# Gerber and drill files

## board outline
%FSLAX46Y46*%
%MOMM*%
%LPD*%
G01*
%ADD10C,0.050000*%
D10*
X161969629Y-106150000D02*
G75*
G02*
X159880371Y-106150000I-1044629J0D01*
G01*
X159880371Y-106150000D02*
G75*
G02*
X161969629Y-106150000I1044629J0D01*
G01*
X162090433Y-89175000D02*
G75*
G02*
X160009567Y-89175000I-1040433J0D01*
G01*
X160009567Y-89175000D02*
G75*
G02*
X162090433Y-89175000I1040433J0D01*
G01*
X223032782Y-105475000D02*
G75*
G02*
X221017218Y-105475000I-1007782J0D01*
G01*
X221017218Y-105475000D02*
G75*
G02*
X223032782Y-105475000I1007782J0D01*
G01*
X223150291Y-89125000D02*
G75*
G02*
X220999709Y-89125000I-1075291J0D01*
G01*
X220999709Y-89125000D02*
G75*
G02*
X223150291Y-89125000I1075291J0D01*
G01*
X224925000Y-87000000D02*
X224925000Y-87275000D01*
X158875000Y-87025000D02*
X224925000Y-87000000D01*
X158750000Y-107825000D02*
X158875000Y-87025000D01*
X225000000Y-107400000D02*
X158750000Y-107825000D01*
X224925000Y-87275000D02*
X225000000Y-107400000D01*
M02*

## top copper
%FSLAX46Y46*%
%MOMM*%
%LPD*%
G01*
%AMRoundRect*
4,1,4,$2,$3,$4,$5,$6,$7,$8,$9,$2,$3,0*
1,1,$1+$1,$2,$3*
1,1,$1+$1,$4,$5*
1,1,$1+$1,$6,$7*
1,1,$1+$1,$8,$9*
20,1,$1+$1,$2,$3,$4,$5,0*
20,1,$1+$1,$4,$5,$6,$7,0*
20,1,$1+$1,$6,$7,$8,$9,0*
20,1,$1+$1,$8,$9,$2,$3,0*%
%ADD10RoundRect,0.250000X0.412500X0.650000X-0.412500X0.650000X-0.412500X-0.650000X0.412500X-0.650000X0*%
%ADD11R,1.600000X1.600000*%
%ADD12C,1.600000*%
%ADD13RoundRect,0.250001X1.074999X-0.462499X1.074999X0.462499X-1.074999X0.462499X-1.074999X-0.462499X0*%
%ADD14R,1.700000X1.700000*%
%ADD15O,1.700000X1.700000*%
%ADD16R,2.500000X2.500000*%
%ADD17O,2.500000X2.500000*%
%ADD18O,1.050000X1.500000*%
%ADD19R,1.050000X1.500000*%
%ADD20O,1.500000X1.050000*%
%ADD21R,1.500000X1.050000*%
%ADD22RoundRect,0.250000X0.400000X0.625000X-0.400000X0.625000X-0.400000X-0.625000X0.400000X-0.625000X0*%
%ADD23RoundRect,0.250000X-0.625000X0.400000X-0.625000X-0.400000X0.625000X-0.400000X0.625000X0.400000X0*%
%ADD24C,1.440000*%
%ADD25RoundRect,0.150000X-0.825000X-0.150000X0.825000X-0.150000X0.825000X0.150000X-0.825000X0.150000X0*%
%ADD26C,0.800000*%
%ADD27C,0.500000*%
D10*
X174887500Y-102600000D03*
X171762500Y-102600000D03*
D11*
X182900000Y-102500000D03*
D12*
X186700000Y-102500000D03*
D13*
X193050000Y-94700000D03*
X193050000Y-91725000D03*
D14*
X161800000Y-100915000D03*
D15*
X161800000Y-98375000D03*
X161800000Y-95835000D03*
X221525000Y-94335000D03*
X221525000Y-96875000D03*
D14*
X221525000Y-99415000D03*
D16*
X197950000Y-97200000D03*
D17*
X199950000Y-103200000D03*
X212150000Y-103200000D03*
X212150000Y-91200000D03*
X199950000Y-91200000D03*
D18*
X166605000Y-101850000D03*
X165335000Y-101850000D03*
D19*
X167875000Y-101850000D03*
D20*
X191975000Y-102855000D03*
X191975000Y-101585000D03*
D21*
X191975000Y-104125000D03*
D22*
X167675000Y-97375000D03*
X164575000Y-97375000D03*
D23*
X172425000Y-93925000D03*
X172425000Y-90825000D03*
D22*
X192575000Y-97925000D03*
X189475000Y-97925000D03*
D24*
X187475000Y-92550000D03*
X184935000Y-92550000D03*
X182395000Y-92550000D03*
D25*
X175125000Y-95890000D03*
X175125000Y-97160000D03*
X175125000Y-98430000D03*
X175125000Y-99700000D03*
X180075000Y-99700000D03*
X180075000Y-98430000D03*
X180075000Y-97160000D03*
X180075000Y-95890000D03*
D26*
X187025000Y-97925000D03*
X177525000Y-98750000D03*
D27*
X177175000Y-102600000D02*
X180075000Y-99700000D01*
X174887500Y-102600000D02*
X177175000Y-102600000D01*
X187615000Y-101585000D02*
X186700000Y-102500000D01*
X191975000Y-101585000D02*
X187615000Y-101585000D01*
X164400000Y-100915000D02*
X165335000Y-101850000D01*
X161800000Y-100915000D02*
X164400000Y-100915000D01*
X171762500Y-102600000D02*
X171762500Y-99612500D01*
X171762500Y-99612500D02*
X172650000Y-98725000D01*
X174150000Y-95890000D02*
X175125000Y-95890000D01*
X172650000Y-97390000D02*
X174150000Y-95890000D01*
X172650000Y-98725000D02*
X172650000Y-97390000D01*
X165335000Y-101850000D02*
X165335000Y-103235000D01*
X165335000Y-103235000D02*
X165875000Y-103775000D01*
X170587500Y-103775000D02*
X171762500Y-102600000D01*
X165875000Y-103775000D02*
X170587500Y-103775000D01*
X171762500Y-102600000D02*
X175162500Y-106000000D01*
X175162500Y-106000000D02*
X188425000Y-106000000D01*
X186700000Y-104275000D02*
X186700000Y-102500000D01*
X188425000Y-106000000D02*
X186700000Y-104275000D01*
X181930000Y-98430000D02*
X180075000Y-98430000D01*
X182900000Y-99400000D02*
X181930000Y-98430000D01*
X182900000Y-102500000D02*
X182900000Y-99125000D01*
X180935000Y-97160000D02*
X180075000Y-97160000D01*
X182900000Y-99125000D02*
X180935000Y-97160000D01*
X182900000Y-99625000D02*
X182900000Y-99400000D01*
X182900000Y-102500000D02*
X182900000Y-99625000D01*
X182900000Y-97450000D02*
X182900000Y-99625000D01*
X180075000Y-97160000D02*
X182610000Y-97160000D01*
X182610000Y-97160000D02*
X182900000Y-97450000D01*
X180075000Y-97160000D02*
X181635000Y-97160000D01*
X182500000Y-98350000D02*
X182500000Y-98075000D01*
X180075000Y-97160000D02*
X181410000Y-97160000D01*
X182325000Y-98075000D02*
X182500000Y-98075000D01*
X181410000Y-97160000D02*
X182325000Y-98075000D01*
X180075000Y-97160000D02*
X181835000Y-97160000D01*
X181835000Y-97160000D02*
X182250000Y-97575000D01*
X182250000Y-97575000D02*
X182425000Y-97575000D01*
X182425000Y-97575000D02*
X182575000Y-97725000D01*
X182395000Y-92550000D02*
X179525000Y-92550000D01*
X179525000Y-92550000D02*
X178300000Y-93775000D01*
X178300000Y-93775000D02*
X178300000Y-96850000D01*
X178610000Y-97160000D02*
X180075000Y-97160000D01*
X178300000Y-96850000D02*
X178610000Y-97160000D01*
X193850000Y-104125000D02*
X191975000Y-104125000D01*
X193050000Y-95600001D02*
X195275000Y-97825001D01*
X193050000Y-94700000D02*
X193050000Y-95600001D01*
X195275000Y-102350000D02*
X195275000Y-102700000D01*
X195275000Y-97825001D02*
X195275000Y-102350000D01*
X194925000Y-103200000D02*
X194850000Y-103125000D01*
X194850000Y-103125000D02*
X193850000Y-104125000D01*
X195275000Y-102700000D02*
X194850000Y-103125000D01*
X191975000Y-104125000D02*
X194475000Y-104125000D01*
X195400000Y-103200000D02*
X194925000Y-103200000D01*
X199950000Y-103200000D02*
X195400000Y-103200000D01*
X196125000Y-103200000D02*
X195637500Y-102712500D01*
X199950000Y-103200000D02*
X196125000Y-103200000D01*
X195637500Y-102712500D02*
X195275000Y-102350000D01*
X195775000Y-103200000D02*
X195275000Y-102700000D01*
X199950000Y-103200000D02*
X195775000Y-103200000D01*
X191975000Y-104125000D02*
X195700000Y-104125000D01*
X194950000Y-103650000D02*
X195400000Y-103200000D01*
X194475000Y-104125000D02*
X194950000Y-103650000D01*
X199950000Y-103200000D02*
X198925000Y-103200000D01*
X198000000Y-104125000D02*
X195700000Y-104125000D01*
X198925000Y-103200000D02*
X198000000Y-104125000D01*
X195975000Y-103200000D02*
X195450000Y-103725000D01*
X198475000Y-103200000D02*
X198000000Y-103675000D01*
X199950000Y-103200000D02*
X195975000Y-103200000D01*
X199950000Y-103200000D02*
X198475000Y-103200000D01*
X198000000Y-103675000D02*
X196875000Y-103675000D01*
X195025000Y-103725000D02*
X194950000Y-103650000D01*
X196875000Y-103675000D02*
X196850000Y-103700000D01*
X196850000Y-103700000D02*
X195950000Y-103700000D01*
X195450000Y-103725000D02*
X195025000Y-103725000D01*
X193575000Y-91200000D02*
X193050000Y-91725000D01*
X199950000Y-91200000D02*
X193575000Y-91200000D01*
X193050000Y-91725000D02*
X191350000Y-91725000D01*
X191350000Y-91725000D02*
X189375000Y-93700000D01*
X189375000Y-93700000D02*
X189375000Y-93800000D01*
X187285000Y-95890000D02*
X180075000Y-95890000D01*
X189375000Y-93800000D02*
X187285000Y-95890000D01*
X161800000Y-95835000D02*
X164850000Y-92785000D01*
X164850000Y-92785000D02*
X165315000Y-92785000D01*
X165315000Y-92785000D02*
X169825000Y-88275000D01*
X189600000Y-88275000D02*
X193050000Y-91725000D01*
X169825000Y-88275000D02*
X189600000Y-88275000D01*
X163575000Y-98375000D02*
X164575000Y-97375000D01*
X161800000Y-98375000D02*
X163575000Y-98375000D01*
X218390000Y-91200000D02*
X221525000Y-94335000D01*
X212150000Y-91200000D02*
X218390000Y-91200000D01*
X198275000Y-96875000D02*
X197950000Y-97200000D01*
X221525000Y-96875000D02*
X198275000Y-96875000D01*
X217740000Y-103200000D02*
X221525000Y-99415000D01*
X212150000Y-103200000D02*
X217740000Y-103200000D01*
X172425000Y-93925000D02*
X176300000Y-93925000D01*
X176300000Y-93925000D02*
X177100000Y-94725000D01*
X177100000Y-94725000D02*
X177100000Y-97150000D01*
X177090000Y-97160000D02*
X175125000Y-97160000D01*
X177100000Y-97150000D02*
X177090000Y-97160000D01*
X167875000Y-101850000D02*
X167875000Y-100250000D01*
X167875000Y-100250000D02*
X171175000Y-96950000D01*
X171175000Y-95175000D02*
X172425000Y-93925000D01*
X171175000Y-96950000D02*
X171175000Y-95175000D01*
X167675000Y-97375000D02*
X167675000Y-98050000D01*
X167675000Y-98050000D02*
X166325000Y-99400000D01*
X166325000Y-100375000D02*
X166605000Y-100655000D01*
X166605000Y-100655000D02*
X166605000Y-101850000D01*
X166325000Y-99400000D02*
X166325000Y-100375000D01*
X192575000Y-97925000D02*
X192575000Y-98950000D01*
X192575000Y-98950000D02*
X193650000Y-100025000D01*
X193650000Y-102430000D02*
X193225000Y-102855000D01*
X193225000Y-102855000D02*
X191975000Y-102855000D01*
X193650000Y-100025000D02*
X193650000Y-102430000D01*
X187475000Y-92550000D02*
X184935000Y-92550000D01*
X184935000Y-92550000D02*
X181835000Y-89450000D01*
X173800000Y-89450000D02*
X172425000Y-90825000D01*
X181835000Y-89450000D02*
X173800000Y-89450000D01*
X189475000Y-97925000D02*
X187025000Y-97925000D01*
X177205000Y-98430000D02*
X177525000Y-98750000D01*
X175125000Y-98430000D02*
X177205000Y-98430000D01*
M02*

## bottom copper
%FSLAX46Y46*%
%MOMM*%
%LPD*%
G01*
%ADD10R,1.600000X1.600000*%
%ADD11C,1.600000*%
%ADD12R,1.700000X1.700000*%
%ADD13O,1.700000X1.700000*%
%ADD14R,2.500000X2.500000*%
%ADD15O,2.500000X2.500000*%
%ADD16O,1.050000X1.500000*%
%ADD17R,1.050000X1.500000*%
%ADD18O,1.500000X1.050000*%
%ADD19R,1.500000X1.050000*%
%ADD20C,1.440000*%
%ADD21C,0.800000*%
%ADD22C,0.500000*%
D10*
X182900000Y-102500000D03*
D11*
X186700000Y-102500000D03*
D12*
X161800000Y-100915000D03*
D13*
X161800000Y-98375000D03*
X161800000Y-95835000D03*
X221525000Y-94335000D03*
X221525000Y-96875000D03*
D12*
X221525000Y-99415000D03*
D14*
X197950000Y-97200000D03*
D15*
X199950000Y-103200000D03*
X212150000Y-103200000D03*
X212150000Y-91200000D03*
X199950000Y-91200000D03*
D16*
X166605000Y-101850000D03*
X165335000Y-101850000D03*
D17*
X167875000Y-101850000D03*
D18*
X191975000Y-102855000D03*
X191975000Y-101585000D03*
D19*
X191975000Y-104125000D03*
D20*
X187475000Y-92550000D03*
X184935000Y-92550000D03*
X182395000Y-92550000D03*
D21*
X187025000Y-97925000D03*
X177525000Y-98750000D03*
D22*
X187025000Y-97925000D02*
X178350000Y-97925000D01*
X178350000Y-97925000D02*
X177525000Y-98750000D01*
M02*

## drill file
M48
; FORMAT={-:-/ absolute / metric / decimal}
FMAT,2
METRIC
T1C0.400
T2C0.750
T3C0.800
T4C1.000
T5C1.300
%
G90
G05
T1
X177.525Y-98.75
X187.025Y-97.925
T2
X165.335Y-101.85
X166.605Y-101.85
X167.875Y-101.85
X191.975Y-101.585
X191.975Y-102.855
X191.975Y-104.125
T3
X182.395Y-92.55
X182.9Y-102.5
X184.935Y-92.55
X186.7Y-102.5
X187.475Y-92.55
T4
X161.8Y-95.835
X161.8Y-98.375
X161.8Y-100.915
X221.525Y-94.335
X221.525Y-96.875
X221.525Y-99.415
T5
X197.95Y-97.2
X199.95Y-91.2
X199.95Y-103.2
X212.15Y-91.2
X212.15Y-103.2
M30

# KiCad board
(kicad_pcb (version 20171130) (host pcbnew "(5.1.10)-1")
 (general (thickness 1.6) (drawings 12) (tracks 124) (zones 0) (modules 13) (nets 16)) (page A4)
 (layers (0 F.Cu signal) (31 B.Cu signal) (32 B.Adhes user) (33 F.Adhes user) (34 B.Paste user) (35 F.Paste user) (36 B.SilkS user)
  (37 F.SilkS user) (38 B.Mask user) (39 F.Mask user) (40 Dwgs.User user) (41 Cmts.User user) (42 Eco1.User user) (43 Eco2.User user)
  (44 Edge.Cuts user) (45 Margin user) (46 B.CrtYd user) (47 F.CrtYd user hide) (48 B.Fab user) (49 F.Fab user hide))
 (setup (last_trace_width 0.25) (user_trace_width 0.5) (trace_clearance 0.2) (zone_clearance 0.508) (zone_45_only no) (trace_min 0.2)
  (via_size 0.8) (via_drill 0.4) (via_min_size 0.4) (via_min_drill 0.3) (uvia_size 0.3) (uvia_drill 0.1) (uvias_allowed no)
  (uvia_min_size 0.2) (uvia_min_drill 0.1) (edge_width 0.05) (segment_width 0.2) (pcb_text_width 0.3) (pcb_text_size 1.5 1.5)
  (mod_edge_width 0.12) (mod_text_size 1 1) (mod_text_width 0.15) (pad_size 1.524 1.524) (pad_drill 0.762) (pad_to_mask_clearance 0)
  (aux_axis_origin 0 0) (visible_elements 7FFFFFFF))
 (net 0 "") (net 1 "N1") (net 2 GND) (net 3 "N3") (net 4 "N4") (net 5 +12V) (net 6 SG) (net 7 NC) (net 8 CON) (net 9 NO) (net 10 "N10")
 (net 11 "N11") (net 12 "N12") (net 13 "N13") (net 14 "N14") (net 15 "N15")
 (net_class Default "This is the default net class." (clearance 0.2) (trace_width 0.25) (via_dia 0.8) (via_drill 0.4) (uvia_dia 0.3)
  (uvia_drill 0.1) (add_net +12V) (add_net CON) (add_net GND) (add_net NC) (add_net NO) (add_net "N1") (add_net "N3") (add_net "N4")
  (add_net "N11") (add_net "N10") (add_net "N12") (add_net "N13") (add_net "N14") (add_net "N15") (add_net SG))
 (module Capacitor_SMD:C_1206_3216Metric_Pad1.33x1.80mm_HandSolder (layer F.Cu) (at 173.325 102.6 180)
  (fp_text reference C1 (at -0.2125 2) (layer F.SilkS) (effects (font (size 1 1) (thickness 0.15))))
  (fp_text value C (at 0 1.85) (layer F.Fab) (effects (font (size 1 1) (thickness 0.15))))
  (pad 1 smd roundrect (at -1.5625 0 180) (size 1.325 1.8) (layers F.Cu F.Paste F.Mask) (roundrect_rratio 0.188679) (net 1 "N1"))
  (pad 2 smd roundrect (at 1.5625 0 180) (size 1.325 1.8) (layers F.Cu F.Paste F.Mask) (roundrect_rratio 0.188679) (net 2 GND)))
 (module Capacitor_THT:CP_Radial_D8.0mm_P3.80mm (layer F.Cu) (at 182.9 102.5)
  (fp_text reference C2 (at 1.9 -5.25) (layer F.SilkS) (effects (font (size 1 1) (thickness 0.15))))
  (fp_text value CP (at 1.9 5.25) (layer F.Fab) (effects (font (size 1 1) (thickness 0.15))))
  (pad 1 thru_hole rect (at 0 0) (size 1.6 1.6) (drill 0.8) (layers *.Cu *.Mask) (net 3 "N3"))
  (pad 2 thru_hole circle (at 3.8 0) (size 1.6 1.6) (drill 0.8) (layers *.Cu *.Mask) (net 2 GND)))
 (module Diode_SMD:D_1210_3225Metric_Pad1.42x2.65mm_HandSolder (layer F.Cu) (at 193.05 93.2125 90)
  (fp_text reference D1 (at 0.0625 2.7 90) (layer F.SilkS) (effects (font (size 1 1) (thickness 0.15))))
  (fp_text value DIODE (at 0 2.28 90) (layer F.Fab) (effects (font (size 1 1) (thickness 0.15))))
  (pad 1 smd roundrect (at -1.4875 0 90) (size 1.425 2.65) (layers F.Cu F.Paste F.Mask) (roundrect_rratio 0.175439) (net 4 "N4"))
  (pad 2 smd roundrect (at 1.4875 0 90) (size 1.425 2.65) (layers F.Cu F.Paste F.Mask) (roundrect_rratio 0.175439) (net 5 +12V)))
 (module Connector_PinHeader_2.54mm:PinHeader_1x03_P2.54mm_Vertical (layer F.Cu) (at 161.8 100.915 180)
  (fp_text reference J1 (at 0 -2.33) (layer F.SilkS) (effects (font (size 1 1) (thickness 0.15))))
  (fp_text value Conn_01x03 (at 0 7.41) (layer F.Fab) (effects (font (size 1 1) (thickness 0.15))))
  (pad 1 thru_hole rect (at 0 0 180) (size 1.7 1.7) (drill 1) (layers *.Cu *.Mask) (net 2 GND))
  (pad 2 thru_hole oval (at 0 2.54 180) (size 1.7 1.7) (drill 1) (layers *.Cu *.Mask) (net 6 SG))
  (pad 3 thru_hole oval (at 0 5.08 180) (size 1.7 1.7) (drill 1) (layers *.Cu *.Mask) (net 5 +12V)))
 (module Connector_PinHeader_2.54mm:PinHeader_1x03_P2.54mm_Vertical (layer F.Cu) (at 221.525 99.415 180)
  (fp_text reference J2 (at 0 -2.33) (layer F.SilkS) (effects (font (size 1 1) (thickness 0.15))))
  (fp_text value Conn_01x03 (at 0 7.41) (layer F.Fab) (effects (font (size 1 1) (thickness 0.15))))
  (pad 3 thru_hole oval (at 0 5.08 180) (size 1.7 1.7) (drill 1) (layers *.Cu *.Mask) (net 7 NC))
  (pad 2 thru_hole oval (at 0 2.54 180) (size 1.7 1.7) (drill 1) (layers *.Cu *.Mask) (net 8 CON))
  (pad 1 thru_hole rect (at 0 0 180) (size 1.7 1.7) (drill 1) (layers *.Cu *.Mask) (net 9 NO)))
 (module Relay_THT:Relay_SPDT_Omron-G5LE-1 (layer F.Cu) (at 197.95 97.2 90)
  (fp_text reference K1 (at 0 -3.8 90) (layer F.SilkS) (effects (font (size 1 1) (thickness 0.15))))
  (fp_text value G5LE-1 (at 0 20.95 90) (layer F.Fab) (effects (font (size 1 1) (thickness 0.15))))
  (pad 1 thru_hole rect (at 0 0 90) (size 2.5 2.5) (drill 1.3) (layers *.Cu *.Mask) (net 8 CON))
  (pad 2 thru_hole oval (at -6 2 90) (size 2.5 2.5) (drill 1.3) (layers *.Cu *.Mask) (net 4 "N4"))
  (pad 3 thru_hole oval (at -6 14.2 90) (size 2.5 2.5) (drill 1.3) (layers *.Cu *.Mask) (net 9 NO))
  (pad 4 thru_hole oval (at 6 14.2 90) (size 2.5 2.5) (drill 1.3) (layers *.Cu *.Mask) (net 7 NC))
  (pad 5 thru_hole oval (at 6 2 90) (size 2.5 2.5) (drill 1.3) (layers *.Cu *.Mask) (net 5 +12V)))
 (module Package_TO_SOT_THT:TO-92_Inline (layer F.Cu) (at 167.875 101.85 180)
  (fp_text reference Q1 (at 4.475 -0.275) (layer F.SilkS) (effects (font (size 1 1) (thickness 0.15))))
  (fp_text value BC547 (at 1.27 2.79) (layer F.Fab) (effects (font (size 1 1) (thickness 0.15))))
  (pad 2 thru_hole oval (at 1.27 0 180) (size 1.05 1.5) (drill 0.75) (layers *.Cu *.Mask) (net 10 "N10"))
  (pad 3 thru_hole oval (at 2.54 0 180) (size 1.05 1.5) (drill 0.75) (layers *.Cu *.Mask) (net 2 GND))
  (pad 1 thru_hole rect (at 0 0 180) (size 1.05 1.5) (drill 0.75) (layers *.Cu *.Mask) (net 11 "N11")))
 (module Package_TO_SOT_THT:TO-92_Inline (layer F.Cu) (at 191.975 104.125 90)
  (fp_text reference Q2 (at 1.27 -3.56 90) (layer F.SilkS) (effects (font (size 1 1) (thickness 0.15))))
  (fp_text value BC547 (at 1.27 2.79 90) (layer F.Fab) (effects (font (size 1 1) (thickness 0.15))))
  (pad 2 thru_hole oval (at 1.27 0 90) (size 1.05 1.5) (drill 0.75) (layers *.Cu *.Mask) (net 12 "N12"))
  (pad 3 thru_hole oval (at 2.54 0 90) (size 1.05 1.5) (drill 0.75) (layers *.Cu *.Mask) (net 2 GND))
  (pad 1 thru_hole rect (at 0 0 90) (size 1.05 1.5) (drill 0.75) (layers *.Cu *.Mask) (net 4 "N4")))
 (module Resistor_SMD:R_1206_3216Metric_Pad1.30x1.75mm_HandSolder (layer F.Cu) (at 166.125 97.375 180)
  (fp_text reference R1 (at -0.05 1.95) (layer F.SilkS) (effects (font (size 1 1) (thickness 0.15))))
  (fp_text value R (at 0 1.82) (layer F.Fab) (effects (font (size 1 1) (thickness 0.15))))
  (pad 1 smd roundrect (at -1.55 0 180) (size 1.3 1.75) (layers F.Cu F.Paste F.Mask) (roundrect_rratio 0.192308) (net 10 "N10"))
  (pad 2 smd roundrect (at 1.55 0 180) (size 1.3 1.75) (layers F.Cu F.Paste F.Mask) (roundrect_rratio 0.192308) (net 6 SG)))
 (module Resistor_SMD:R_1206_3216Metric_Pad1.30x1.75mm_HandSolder (layer F.Cu) (at 172.425 92.375 270)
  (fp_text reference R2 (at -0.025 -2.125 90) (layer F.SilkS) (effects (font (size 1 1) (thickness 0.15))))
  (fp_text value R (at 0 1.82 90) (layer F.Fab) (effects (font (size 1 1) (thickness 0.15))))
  (pad 2 smd roundrect (at 1.55 0 270) (size 1.3 1.75) (layers F.Cu F.Paste F.Mask) (roundrect_rratio 0.192308) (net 11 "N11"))
  (pad 1 smd roundrect (at -1.55 0 270) (size 1.3 1.75) (layers F.Cu F.Paste F.Mask) (roundrect_rratio 0.192308) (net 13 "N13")))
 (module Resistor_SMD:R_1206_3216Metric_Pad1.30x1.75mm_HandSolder (layer F.Cu) (at 191.025 97.925 180)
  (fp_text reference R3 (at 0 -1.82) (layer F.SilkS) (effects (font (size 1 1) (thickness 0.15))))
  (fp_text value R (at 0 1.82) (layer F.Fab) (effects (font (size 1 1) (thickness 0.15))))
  (pad 1 smd roundrect (at -1.55 0 180) (size 1.3 1.75) (layers F.Cu F.Paste F.Mask) (roundrect_rratio 0.192308) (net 12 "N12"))
  (pad 2 smd roundrect (at 1.55 0 180) (size 1.3 1.75) (layers F.Cu F.Paste F.Mask) (roundrect_rratio 0.192308) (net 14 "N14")))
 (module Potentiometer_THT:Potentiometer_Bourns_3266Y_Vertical (layer F.Cu) (at 187.475 92.55)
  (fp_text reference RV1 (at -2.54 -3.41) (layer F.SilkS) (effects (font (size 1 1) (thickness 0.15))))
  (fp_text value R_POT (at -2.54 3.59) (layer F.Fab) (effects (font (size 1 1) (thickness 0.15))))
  (pad 1 thru_hole circle (at 0 0) (size 1.44 1.44) (drill 0.8) (layers *.Cu *.Mask) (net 13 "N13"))
  (pad 2 thru_hole circle (at -2.54 0) (size 1.44 1.44) (drill 0.8) (layers *.Cu *.Mask) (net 13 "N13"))
  (pad 3 thru_hole circle (at -5.08 0) (size 1.44 1.44) (drill 0.8) (layers *.Cu *.Mask) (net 3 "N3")))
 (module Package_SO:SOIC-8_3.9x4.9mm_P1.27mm (layer F.Cu) (at 177.6 97.795)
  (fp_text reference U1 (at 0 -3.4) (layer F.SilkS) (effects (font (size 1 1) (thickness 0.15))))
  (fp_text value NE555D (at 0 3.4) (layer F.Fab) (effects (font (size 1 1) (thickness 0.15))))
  (pad 1 smd roundrect (at -2.475 -1.905) (size 1.95 0.6) (layers F.Cu F.Paste F.Mask) (roundrect_rratio 0.25) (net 2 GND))
  (pad 2 smd roundrect (at -2.475 -0.635) (size 1.95 0.6) (layers F.Cu F.Paste F.Mask) (roundrect_rratio 0.25) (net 11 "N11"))
  (pad 3 smd roundrect (at -2.475 0.635) (size 1.95 0.6) (layers F.Cu F.Paste F.Mask) (roundrect_rratio 0.25) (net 14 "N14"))
  (pad 4 smd roundrect (at -2.475 1.905) (size 1.95 0.6) (layers F.Cu F.Paste F.Mask) (roundrect_rratio 0.25) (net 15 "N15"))
  (pad 5 smd roundrect (at 2.475 1.905) (size 1.95 0.6) (layers F.Cu F.Paste F.Mask) (roundrect_rratio 0.25) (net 1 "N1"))
  (pad 6 smd roundrect (at 2.475 0.635) (size 1.95 0.6) (layers F.Cu F.Paste F.Mask) (roundrect_rratio 0.25) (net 3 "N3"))
  (pad 7 smd roundrect (at 2.475 -0.635) (size 1.95 0.6) (layers F.Cu F.Paste F.Mask) (roundrect_rratio 0.25) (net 3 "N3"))
  (pad 8 smd roundrect (at 2.475 -1.905) (size 1.95 0.6) (layers F.Cu F.Paste F.Mask) (roundrect_rratio 0.25) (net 5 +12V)))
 (gr_circle (center 160.925 106.15) (end 161.9 105.775) (layer Edge.Cuts) (width 0.05))
 (gr_circle (center 161.05 89.175) (end 161.9 88.575) (layer Edge.Cuts) (width 0.05))
 (gr_circle (center 222.025 105.475) (end 222.75 104.775) (layer Edge.Cuts) (width 0.05))
 (gr_circle (center 222.075 89.125) (end 222.7 88.25) (layer Edge.Cuts) (width 0.05))
 (gr_line (start 224.925 87) (end 224.925 87.275) (layer Edge.Cuts) (width 0.05))
 (gr_line (start 158.875 87.025) (end 224.925 87) (layer Edge.Cuts) (width 0.05))
 (gr_line (start 158.75 107.825) (end 158.875 87.025) (layer Edge.Cuts) (width 0.05))
 (gr_line (start 225 107.4) (end 158.75 107.825) (layer Edge.Cuts) (width 0.05))
 (gr_line (start 224.925 87.275) (end 225 107.4) (layer Edge.Cuts) (width 0.05))
 (segment (start 177.175 102.6) (end 180.075 99.7) (width 0.5) (layer F.Cu) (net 1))
 (segment (start 174.8875 102.6) (end 177.175 102.6) (width 0.5) (layer F.Cu) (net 1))
 (segment (start 187.615 101.585) (end 186.7 102.5) (width 0.5) (layer F.Cu) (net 2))
 (segment (start 191.975 101.585) (end 187.615 101.585) (width 0.5) (layer F.Cu) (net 2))
 (segment (start 164.4 100.915) (end 165.335 101.85) (width 0.5) (layer F.Cu) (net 2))
 (segment (start 161.8 100.915) (end 164.4 100.915) (width 0.5) (layer F.Cu) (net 2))
 (segment (start 171.7625 102.6) (end 171.7625 99.6125) (width 0.5) (layer F.Cu) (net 2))
 (segment (start 171.7625 99.6125) (end 172.65 98.725) (width 0.5) (layer F.Cu) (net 2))
 (segment (start 174.15 95.89) (end 175.125 95.89) (width 0.5) (layer F.Cu) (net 2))
 (segment (start 172.65 97.39) (end 174.15 95.89) (width 0.5) (layer F.Cu) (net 2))
 (segment (start 172.65 98.725) (end 172.65 97.39) (width 0.5) (layer F.Cu) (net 2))
 (segment (start 165.335 101.85) (end 165.335 103.235) (width 0.5) (layer F.Cu) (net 2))
 (segment (start 165.335 103.235) (end 165.875 103.775) (width 0.5) (layer F.Cu) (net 2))
 (segment (start 170.5875 103.775) (end 171.7625 102.6) (width 0.5) (layer F.Cu) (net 2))
 (segment (start 165.875 103.775) (end 170.5875 103.775) (width 0.5) (layer F.Cu) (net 2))
 (segment (start 171.7625 102.6) (end 175.1625 106) (width 0.5) (layer F.Cu) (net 2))
 (segment (start 175.1625 106) (end 188.425 106) (width 0.5) (layer F.Cu) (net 2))
 (segment (start 186.7 104.275) (end 186.7 102.5) (width 0.5) (layer F.Cu) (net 2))
 (segment (start 188.425 106) (end 186.7 104.275) (width 0.5) (layer F.Cu) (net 2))
 (segment (start 181.93 98.43) (end 180.075 98.43) (width 0.5) (layer F.Cu) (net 3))
 (segment (start 182.9 99.4) (end 181.93 98.43) (width 0.5) (layer F.Cu) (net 3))
 (segment (start 182.9 102.5) (end 182.9 99.125) (width 0.5) (layer F.Cu) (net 3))
 (segment (start 180.935 97.16) (end 180.075 97.16) (width 0.5) (layer F.Cu) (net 3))
 (segment (start 182.9 99.125) (end 180.935 97.16) (width 0.5) (layer F.Cu) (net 3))
 (segment (start 182.9 99.625) (end 182.9 99.4) (width 0.5) (layer F.Cu) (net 3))
 (segment (start 182.9 102.5) (end 182.9 99.625) (width 0.5) (layer F.Cu) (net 3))
 (segment (start 182.9 97.45) (end 182.9 99.625) (width 0.5) (layer F.Cu) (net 3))
 (segment (start 180.075 97.16) (end 182.61 97.16) (width 0.5) (layer F.Cu) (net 3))
 (segment (start 182.61 97.16) (end 182.9 97.45) (width 0.5) (layer F.Cu) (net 3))
 (segment (start 180.075 97.16) (end 181.635 97.16) (width 0.5) (layer F.Cu) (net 3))
 (segment (start 182.5 98.35) (end 182.5 98.075) (width 0.5) (layer F.Cu) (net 3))
 (segment (start 180.075 97.16) (end 181.41 97.16) (width 0.5) (layer F.Cu) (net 3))
 (segment (start 182.325 98.075) (end 182.5 98.075) (width 0.5) (layer F.Cu) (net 3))
 (segment (start 181.41 97.16) (end 182.325 98.075) (width 0.5) (layer F.Cu) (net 3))
 (segment (start 180.075 97.16) (end 181.835 97.16) (width 0.5) (layer F.Cu) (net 3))
 (segment (start 181.835 97.16) (end 182.25 97.575) (width 0.5) (layer F.Cu) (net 3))
 (segment (start 182.25 97.575) (end 182.425 97.575) (width 0.5) (layer F.Cu) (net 3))
 (segment (start 182.425 97.575) (end 182.575 97.725) (width 0.5) (layer F.Cu) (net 3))
 (segment (start 182.395 92.55) (end 179.525 92.55) (width 0.5) (layer F.Cu) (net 3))
 (segment (start 179.525 92.55) (end 178.3 93.775) (width 0.5) (layer F.Cu) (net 3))
 (segment (start 178.3 93.775) (end 178.3 96.85) (width 0.5) (layer F.Cu) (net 3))
 (segment (start 178.61 97.16) (end 180.075 97.16) (width 0.5) (layer F.Cu) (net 3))
 (segment (start 178.3 96.85) (end 178.61 97.16) (width 0.5) (layer F.Cu) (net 3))
 (segment (start 193.85 104.125) (end 191.975 104.125) (width 0.5) (layer F.Cu) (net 4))
 (segment (start 193.05 95.600001) (end 195.275 97.825001) (width 0.5) (layer F.Cu) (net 4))
 (segment (start 193.05 94.7) (end 193.05 95.600001) (width 0.5) (layer F.Cu) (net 4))
 (segment (start 195.275 102.35) (end 195.275 102.7) (width 0.5) (layer F.Cu) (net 4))
 (segment (start 195.275 97.825001) (end 195.275 102.35) (width 0.5) (layer F.Cu) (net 4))
 (segment (start 194.925 103.2) (end 194.85 103.125) (width 0.5) (layer F.Cu) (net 4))
 (segment (start 194.85 103.125) (end 193.85 104.125) (width 0.5) (layer F.Cu) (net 4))
 (segment (start 195.275 102.7) (end 194.85 103.125) (width 0.5) (layer F.Cu) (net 4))
 (segment (start 191.975 104.125) (end 194.475 104.125) (width 0.5) (layer F.Cu) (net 4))
 (segment (start 195.4 103.2) (end 194.925 103.2) (width 0.5) (layer F.Cu) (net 4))
 (segment (start 199.95 103.2) (end 195.4 103.2) (width 0.5) (layer F.Cu) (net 4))
 (segment (start 196.125 103.2) (end 195.6375 102.7125) (width 0.5) (layer F.Cu) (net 4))
 (segment (start 199.95 103.2) (end 196.125 103.2) (width 0.5) (layer F.Cu) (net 4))
 (segment (start 195.6375 102.7125) (end 195.275 102.35) (width 0.5) (layer F.Cu) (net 4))
 (segment (start 195.775 103.2) (end 195.275 102.7) (width 0.5) (layer F.Cu) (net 4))
 (segment (start 199.95 103.2) (end 195.775 103.2) (width 0.5) (layer F.Cu) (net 4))
 (segment (start 191.975 104.125) (end 195.7 104.125) (width 0.5) (layer F.Cu) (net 4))
 (segment (start 194.95 103.65) (end 195.4 103.2) (width 0.5) (layer F.Cu) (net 4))
 (segment (start 194.475 104.125) (end 194.95 103.65) (width 0.5) (layer F.Cu) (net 4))
 (segment (start 199.95 103.2) (end 198.925 103.2) (width 0.5) (layer F.Cu) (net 4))
 (segment (start 198 104.125) (end 195.7 104.125) (width 0.5) (layer F.Cu) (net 4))
 (segment (start 198.925 103.2) (end 198 104.125) (width 0.5) (layer F.Cu) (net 4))
 (segment (start 195.975 103.2) (end 195.45 103.725) (width 0.5) (layer F.Cu) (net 4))
 (segment (start 198.475 103.2) (end 198 103.675) (width 0.5) (layer F.Cu) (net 4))
 (segment (start 199.95 103.2) (end 195.975 103.2) (width 0.5) (layer F.Cu) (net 4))
 (segment (start 199.95 103.2) (end 198.475 103.2) (width 0.5) (layer F.Cu) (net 4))
 (segment (start 198 103.675) (end 196.875 103.675) (width 0.5) (layer F.Cu) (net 4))
 (segment (start 195.025 103.725) (end 194.95 103.65) (width 0.5) (layer F.Cu) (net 4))
 (segment (start 196.875 103.675) (end 196.85 103.7) (width 0.5) (layer F.Cu) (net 4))
 (segment (start 196.85 103.7) (end 195.95 103.7) (width 0.5) (layer F.Cu) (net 4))
 (segment (start 195.45 103.725) (end 195.025 103.725) (width 0.5) (layer F.Cu) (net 4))
 (segment (start 193.575 91.2) (end 193.05 91.725) (width 0.5) (layer F.Cu) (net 5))
 (segment (start 199.95 91.2) (end 193.575 91.2) (width 0.5) (layer F.Cu) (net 5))
 (segment (start 193.05 91.725) (end 191.35 91.725) (width 0.5) (layer F.Cu) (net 5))
 (segment (start 191.35 91.725) (end 189.375 93.7) (width 0.5) (layer F.Cu) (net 5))
 (segment (start 189.375 93.7) (end 189.375 93.8) (width 0.5) (layer F.Cu) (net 5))
 (segment (start 187.285 95.89) (end 180.075 95.89) (width 0.5) (layer F.Cu) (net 5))
 (segment (start 189.375 93.8) (end 187.285 95.89) (width 0.5) (layer F.Cu) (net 5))
 (segment (start 161.8 95.835) (end 164.85 92.785) (width 0.5) (layer F.Cu) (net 5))
 (segment (start 164.85 92.785) (end 165.315 92.785) (width 0.5) (layer F.Cu) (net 5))
 (segment (start 165.315 92.785) (end 169.825 88.275) (width 0.5) (layer F.Cu) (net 5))
 (segment (start 189.6 88.275) (end 193.05 91.725) (width 0.5) (layer F.Cu) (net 5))
 (segment (start 169.825 88.275) (end 189.6 88.275) (width 0.5) (layer F.Cu) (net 5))
 (segment (start 163.575 98.375) (end 164.575 97.375) (width 0.5) (layer F.Cu) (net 6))
 (segment (start 161.8 98.375) (end 163.575 98.375) (width 0.5) (layer F.Cu) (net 6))
 (segment (start 218.39 91.2) (end 221.525 94.335) (width 0.5) (layer F.Cu) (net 7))
 (segment (start 212.15 91.2) (end 218.39 91.2) (width 0.5) (layer F.Cu) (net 7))
 (segment (start 198.275 96.875) (end 197.95 97.2) (width 0.5) (layer F.Cu) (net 8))
 (segment (start 221.525 96.875) (end 198.275 96.875) (width 0.5) (layer F.Cu) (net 8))
 (segment (start 217.74 103.2) (end 221.525 99.415) (width 0.5) (layer F.Cu) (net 9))
 (segment (start 212.15 103.2) (end 217.74 103.2) (width 0.5) (layer F.Cu) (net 9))
 (segment (start 172.425 93.925) (end 176.3 93.925) (width 0.5) (layer F.Cu) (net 11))
 (segment (start 176.3 93.925) (end 177.1 94.725) (width 0.5) (layer F.Cu) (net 11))
 (segment (start 177.1 94.725) (end 177.1 97.15) (width 0.5) (layer F.Cu) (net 11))
 (segment (start 177.09 97.16) (end 175.125 97.16) (width 0.5) (layer F.Cu) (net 11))
 (segment (start 177.1 97.15) (end 177.09 97.16) (width 0.5) (layer F.Cu) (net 11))
 (segment (start 167.875 101.85) (end 167.875 100.25) (width 0.5) (layer F.Cu) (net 11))
 (segment (start 167.875 100.25) (end 171.175 96.95) (width 0.5) (layer F.Cu) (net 11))
 (segment (start 171.175 95.175) (end 172.425 93.925) (width 0.5) (layer F.Cu) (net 11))
 (segment (start 171.175 96.95) (end 171.175 95.175) (width 0.5) (layer F.Cu) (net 11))
 (segment (start 167.675 97.375) (end 167.675 98.05) (width 0.5) (layer F.Cu) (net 10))
 (segment (start 167.675 98.05) (end 166.325 99.4) (width 0.5) (layer F.Cu) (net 10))
 (segment (start 166.325 100.375) (end 166.605 100.655) (width 0.5) (layer F.Cu) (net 10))
 (segment (start 166.605 100.655) (end 166.605 101.85) (width 0.5) (layer F.Cu) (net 10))
 (segment (start 166.325 99.4) (end 166.325 100.375) (width 0.5) (layer F.Cu) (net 10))
 (segment (start 192.575 97.925) (end 192.575 98.95) (width 0.5) (layer F.Cu) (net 12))
 (segment (start 192.575 98.95) (end 193.65 100.025) (width 0.5) (layer F.Cu) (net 12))
 (segment (start 193.65 102.43) (end 193.225 102.855) (width 0.5) (layer F.Cu) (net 12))
 (segment (start 193.225 102.855) (end 191.975 102.855) (width 0.5) (layer F.Cu) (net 12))
 (segment (start 193.65 100.025) (end 193.65 102.43) (width 0.5) (layer F.Cu) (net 12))
 (segment (start 187.475 92.55) (end 184.935 92.55) (width 0.5) (layer F.Cu) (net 13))
 (segment (start 184.935 92.55) (end 181.835 89.45) (width 0.5) (layer F.Cu) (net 13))
 (segment (start 173.8 89.45) (end 172.425 90.825) (width 0.5) (layer F.Cu) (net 13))
 (segment (start 181.835 89.45) (end 173.8 89.45) (width 0.5) (layer F.Cu) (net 13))
 (segment (start 189.475 97.925) (end 187.025 97.925) (width 0.5) (layer F.Cu) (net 14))
 (via (at 187.025 97.925) (size 0.8) (drill 0.4) (layers F.Cu B.Cu) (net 14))
 (segment (start 187.025 97.925) (end 178.35 97.925) (width 0.5) (layer B.Cu) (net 14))
 (via (at 177.525 98.75) (size 0.8) (drill 0.4) (layers F.Cu B.Cu) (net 14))
 (segment (start 178.35 97.925) (end 177.525 98.75) (width 0.5) (layer B.Cu) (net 14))
 (segment (start 177.205 98.43) (end 177.525 98.75) (width 0.5) (layer F.Cu) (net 14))
 (segment (start 175.125 98.43) (end 177.205 98.43) (width 0.5) (layer F.Cu) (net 14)))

